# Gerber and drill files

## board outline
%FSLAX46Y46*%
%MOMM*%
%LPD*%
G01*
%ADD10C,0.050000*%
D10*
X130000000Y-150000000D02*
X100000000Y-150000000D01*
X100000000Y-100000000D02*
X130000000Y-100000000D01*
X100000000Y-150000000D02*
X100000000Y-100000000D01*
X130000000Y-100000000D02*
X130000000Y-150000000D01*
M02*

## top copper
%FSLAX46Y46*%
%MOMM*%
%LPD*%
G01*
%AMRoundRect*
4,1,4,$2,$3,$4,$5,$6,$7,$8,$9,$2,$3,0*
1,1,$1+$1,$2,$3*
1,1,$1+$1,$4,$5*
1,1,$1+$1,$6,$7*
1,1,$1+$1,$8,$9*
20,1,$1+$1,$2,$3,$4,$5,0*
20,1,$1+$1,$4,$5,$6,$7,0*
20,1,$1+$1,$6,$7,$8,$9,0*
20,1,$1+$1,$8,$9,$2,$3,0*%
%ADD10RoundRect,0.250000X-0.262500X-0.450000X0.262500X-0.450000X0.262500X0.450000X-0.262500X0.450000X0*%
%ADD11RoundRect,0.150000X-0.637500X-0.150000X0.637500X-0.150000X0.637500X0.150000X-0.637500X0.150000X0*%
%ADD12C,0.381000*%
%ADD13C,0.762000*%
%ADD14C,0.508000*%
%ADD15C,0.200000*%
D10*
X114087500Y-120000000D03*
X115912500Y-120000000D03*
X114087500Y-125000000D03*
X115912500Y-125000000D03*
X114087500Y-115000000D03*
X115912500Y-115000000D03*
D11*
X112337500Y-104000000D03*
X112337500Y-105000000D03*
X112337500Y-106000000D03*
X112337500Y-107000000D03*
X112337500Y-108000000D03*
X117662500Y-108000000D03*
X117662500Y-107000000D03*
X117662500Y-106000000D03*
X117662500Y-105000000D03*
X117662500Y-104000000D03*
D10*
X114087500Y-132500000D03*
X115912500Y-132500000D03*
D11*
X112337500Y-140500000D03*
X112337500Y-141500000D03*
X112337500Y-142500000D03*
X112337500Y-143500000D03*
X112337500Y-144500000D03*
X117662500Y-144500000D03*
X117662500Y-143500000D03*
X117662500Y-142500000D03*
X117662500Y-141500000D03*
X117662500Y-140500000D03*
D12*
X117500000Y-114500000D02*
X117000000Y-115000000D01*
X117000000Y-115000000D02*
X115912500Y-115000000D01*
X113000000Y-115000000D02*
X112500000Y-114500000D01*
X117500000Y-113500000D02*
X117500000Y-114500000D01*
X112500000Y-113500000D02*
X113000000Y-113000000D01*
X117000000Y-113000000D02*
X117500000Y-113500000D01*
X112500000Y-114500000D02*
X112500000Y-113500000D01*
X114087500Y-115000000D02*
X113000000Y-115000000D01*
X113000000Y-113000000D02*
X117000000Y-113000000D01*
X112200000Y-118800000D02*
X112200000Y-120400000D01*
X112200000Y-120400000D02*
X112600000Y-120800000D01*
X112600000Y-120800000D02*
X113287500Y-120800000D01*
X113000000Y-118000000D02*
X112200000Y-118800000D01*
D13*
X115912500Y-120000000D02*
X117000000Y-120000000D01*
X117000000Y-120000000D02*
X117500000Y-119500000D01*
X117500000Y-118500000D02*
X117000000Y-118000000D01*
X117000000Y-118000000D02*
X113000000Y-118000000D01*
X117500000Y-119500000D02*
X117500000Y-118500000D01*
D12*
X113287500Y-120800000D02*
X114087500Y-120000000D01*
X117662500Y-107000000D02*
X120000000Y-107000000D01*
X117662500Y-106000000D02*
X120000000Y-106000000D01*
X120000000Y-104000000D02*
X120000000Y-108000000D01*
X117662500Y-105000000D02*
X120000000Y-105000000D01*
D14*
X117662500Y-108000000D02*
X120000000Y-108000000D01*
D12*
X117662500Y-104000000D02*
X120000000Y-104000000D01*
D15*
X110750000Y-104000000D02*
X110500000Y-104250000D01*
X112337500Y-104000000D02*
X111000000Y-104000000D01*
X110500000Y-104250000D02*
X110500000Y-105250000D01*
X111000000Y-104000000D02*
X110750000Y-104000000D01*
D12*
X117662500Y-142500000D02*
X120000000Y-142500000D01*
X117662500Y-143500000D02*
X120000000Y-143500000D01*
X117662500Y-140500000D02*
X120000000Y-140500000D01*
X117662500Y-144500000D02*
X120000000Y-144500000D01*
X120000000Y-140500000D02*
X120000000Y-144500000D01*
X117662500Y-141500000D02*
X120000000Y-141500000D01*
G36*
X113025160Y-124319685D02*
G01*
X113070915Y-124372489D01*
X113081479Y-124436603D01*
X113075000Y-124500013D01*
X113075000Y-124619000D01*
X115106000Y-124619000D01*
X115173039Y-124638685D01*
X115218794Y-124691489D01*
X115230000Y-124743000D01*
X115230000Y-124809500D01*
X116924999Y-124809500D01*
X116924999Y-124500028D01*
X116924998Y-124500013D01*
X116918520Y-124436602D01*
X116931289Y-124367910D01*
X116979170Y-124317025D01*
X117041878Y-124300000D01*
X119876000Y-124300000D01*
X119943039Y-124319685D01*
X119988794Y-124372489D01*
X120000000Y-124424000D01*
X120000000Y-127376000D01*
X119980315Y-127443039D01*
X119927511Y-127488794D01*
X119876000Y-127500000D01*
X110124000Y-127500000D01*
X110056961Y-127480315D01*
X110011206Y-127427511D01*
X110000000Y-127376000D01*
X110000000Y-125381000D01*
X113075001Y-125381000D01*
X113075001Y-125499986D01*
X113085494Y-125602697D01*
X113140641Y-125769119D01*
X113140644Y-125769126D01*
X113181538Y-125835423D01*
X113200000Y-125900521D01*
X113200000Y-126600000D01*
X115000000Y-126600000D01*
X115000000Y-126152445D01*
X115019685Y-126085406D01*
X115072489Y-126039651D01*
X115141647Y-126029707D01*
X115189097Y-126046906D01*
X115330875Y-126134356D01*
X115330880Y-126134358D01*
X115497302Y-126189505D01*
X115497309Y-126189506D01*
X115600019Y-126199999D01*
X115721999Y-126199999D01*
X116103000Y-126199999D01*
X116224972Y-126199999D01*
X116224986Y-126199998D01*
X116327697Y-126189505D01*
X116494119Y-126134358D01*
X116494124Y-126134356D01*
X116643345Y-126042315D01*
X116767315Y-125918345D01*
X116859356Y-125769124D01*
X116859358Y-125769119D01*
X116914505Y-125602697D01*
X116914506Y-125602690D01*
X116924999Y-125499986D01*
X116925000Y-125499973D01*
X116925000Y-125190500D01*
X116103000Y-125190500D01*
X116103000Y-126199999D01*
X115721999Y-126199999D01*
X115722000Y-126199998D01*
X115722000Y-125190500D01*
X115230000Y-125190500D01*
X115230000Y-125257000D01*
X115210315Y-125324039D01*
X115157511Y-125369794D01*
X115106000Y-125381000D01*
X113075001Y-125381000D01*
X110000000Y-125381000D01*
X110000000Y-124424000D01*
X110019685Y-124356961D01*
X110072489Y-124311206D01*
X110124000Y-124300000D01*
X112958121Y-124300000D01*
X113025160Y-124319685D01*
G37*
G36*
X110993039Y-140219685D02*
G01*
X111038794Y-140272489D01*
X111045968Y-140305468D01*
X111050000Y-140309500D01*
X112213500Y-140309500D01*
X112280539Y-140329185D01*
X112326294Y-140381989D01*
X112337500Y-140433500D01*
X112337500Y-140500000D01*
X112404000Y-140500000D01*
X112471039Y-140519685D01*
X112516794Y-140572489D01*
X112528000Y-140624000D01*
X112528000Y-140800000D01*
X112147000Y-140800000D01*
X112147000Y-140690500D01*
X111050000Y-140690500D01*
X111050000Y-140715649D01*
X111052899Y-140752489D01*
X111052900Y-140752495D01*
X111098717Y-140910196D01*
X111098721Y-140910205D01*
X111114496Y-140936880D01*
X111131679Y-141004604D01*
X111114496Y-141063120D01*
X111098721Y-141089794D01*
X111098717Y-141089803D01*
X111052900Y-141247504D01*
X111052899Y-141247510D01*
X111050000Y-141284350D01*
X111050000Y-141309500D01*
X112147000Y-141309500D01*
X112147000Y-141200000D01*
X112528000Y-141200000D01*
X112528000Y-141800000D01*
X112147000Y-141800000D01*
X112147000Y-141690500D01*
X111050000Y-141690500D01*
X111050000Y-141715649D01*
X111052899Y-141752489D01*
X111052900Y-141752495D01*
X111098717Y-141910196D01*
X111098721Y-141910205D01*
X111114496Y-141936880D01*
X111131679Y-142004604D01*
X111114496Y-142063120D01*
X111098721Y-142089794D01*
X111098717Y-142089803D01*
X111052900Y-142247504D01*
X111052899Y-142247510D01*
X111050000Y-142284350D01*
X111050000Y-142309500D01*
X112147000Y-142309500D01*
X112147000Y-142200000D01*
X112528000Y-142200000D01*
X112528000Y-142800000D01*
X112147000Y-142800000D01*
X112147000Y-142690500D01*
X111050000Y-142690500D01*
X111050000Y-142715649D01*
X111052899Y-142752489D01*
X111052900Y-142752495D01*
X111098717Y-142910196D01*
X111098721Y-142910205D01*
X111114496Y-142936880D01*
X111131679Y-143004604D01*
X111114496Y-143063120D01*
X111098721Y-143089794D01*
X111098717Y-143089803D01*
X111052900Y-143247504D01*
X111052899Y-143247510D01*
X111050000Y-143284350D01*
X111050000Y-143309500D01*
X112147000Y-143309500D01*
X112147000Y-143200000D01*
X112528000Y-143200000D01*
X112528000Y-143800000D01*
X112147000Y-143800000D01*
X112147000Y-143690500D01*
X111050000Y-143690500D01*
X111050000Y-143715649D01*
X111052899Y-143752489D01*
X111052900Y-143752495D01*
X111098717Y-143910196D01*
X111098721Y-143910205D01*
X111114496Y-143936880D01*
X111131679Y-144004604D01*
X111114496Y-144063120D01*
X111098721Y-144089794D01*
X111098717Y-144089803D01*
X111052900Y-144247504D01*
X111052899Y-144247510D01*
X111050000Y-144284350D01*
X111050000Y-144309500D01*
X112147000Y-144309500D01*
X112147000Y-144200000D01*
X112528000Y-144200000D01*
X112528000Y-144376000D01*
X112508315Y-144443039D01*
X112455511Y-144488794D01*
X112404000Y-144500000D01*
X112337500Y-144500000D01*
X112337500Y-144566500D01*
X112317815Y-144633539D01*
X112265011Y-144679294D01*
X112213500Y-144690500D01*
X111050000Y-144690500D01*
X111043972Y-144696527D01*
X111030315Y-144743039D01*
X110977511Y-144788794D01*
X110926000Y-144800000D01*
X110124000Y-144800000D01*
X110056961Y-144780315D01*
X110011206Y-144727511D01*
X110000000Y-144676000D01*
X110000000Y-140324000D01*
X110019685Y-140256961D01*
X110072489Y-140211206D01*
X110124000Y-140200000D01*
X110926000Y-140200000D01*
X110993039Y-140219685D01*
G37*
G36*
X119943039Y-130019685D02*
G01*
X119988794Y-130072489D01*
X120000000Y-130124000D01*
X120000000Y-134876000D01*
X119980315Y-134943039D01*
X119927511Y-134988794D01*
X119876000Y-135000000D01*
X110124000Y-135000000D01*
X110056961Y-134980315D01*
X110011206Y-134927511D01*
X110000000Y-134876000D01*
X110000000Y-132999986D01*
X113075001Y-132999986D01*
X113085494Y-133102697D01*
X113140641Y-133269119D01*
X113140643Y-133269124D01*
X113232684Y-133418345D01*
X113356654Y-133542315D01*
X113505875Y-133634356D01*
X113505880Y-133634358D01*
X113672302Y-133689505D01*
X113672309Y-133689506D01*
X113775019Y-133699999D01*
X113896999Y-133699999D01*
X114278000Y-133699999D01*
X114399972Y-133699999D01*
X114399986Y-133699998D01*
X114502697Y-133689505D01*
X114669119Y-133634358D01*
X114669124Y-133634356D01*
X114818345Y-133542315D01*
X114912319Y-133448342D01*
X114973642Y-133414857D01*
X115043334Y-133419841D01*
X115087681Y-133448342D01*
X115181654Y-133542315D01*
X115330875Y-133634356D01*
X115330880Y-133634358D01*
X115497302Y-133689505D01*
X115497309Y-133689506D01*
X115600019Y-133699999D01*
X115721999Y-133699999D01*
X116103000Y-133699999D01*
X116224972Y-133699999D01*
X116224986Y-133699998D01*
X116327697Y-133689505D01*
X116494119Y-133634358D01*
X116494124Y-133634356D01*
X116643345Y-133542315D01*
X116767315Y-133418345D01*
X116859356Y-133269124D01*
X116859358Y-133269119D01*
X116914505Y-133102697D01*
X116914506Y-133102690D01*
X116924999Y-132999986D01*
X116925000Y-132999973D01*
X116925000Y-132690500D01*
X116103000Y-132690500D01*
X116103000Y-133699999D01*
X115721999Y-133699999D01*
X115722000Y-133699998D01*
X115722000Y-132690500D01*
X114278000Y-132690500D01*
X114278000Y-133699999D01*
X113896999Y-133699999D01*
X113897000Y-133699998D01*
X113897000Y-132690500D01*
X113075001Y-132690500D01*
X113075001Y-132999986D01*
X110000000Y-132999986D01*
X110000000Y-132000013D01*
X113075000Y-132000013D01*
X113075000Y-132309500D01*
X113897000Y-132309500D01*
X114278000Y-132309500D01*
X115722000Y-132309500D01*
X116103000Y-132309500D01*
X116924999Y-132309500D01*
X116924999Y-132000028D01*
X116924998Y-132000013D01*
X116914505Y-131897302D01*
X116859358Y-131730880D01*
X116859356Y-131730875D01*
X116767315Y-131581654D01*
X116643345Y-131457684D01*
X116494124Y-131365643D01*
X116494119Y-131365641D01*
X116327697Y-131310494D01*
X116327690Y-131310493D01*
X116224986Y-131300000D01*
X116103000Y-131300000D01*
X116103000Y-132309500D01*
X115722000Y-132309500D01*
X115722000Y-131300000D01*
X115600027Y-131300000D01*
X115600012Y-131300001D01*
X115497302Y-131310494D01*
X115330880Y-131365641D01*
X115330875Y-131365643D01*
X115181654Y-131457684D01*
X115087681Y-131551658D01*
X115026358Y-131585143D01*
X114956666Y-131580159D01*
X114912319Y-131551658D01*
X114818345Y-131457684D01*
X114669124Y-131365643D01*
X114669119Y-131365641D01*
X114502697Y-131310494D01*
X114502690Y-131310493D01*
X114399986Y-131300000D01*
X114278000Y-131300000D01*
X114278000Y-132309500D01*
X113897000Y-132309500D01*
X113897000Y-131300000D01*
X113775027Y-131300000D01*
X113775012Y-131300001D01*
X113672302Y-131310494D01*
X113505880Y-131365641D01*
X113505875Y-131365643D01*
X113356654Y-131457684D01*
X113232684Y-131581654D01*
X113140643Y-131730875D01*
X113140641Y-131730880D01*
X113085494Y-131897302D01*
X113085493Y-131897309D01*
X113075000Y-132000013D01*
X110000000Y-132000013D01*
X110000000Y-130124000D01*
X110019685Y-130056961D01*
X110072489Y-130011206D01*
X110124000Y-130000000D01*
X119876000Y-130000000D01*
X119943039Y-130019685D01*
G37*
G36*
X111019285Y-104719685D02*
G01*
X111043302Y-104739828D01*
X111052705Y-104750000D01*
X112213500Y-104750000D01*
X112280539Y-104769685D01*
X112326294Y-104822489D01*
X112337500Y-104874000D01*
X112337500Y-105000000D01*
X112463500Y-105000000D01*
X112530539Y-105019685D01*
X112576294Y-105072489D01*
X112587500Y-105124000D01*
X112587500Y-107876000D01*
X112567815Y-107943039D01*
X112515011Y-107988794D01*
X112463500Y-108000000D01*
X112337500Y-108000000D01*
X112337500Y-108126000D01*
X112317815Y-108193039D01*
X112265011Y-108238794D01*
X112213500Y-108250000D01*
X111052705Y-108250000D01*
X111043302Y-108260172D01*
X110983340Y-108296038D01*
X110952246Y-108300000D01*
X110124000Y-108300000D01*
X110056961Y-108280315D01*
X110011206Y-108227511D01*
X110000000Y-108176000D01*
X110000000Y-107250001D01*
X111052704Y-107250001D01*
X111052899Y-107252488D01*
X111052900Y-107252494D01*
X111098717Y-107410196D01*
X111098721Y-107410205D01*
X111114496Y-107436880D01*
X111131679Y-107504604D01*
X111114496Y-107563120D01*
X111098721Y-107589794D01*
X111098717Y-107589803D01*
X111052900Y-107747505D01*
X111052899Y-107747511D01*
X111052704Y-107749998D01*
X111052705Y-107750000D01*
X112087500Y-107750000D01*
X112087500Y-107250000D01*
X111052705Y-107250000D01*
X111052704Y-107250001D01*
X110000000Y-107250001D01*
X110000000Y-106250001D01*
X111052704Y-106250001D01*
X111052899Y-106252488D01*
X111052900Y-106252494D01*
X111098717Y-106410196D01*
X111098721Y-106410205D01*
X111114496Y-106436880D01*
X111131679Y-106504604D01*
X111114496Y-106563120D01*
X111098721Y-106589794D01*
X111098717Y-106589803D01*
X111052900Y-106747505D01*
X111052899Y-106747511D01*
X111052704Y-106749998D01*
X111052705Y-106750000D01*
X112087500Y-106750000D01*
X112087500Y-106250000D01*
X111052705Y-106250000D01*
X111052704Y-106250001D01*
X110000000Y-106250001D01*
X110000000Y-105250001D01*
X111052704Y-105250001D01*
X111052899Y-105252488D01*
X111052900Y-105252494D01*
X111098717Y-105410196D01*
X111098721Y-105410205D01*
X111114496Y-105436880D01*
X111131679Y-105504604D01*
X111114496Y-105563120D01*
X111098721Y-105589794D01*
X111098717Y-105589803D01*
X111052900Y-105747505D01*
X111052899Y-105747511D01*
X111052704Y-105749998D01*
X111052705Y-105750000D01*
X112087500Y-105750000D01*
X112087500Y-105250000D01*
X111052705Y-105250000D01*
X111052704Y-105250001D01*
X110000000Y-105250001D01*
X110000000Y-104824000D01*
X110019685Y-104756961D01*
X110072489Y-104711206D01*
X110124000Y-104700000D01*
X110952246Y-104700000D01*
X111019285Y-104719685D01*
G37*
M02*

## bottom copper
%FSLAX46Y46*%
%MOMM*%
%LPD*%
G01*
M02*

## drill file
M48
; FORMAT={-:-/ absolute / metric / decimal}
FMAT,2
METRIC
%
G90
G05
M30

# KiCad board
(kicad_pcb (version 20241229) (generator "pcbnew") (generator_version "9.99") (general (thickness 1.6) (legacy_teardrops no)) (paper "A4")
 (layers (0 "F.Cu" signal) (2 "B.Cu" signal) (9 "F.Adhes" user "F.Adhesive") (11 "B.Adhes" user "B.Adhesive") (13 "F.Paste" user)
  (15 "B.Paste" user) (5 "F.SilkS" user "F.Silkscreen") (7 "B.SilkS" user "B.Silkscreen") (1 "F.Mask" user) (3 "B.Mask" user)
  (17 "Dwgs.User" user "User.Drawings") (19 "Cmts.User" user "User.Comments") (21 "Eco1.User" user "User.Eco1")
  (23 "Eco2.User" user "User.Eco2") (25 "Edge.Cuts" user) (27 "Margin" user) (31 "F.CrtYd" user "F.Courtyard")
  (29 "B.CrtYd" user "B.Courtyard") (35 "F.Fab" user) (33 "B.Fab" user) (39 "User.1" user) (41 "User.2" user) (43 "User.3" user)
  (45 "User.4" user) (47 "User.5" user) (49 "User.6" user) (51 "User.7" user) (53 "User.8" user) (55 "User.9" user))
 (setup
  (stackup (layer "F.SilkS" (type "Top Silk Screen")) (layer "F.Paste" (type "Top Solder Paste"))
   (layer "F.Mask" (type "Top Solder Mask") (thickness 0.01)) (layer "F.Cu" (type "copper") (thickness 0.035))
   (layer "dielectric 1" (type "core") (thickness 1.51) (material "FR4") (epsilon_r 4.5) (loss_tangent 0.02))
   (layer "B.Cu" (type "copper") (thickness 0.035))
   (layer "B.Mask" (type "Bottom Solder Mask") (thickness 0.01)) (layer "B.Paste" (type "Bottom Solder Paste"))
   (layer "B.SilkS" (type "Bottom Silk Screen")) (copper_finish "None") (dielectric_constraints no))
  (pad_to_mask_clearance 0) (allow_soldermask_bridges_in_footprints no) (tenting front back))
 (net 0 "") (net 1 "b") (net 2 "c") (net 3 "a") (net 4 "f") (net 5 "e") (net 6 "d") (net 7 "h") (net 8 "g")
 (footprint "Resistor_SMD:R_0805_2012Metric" (layer "F.Cu") (at 115 120)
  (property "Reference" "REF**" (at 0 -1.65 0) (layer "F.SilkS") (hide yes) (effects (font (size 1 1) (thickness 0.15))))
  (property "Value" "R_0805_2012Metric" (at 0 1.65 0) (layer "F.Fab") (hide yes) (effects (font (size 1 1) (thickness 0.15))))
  (pad "1" smd roundrect (at -0.9125 0) (size 1.025 1.4) (layers "F.Cu" "F.Mask" "F.Paste") (roundrect_rratio 0.243902) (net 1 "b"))
  (pad "2" smd roundrect (at 0.9125 0) (size 1.025 1.4) (layers "F.Cu" "F.Mask" "F.Paste") (roundrect_rratio 0.243902) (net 1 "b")))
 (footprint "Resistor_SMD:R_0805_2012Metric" (layer "F.Cu") (at 115 125)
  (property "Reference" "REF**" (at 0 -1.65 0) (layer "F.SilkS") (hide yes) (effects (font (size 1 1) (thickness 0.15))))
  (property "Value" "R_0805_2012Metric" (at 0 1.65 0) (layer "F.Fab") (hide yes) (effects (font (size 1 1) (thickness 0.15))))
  (pad "1" smd roundrect (at -0.9125 0) (size 1.025 1.4) (layers "F.Cu" "F.Mask" "F.Paste") (roundrect_rratio 0.243902) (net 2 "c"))
  (pad "2" smd roundrect (at 0.9125 0) (size 1.025 1.4) (layers "F.Cu" "F.Mask" "F.Paste") (roundrect_rratio 0.243902) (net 2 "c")
   (thermal_bridge_width 0.381)))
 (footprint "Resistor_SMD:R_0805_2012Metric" (layer "F.Cu") (at 115 115)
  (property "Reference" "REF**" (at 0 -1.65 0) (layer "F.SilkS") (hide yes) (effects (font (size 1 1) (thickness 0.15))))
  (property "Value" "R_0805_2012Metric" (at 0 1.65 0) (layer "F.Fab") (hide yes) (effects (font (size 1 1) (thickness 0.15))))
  (pad "1" smd roundrect (at -0.9125 0) (size 1.025 1.4) (layers "F.Cu" "F.Mask" "F.Paste") (roundrect_rratio 0.243902) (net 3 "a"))
  (pad "2" smd roundrect (at 0.9125 0) (size 1.025 1.4) (layers "F.Cu" "F.Mask" "F.Paste") (roundrect_rratio 0.243902) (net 3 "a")))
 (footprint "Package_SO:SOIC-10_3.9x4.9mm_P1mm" (layer "F.Cu") (at 115 106)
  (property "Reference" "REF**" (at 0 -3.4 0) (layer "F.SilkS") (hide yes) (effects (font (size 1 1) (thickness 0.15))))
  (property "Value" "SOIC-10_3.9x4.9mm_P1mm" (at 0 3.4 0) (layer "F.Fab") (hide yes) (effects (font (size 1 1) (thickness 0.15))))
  (pad "1" smd roundrect (at -2.6625 -2) (size 1.575 0.6) (layers "F.Cu" "F.Mask" "F.Paste") (roundrect_rratio 0.25) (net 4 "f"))
  (pad "2" smd roundrect (at -2.6625 -1) (size 1.575 0.6) (layers "F.Cu" "F.Mask" "F.Paste") (roundrect_rratio 0.25) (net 4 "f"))
  (pad "3" smd roundrect (at -2.6625 0) (size 1.575 0.6) (layers "F.Cu" "F.Mask" "F.Paste") (roundrect_rratio 0.25) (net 4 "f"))
  (pad "4" smd roundrect (at -2.6625 1) (size 1.575 0.6) (layers "F.Cu" "F.Mask" "F.Paste") (roundrect_rratio 0.25) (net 4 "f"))
  (pad "5" smd roundrect (at -2.6625 2) (size 1.575 0.6) (layers "F.Cu" "F.Mask" "F.Paste") (roundrect_rratio 0.25) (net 4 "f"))
  (pad "6" smd roundrect (at 2.6625 2) (size 1.575 0.6) (layers "F.Cu" "F.Mask" "F.Paste") (roundrect_rratio 0.25) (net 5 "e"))
  (pad "7" smd roundrect (at 2.6625 1) (size 1.575 0.6) (layers "F.Cu" "F.Mask" "F.Paste") (roundrect_rratio 0.25) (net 5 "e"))
  (pad "8" smd roundrect (at 2.6625 0) (size 1.575 0.6) (layers "F.Cu" "F.Mask" "F.Paste") (roundrect_rratio 0.25) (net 5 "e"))
  (pad "9" smd roundrect (at 2.6625 -1) (size 1.575 0.6) (layers "F.Cu" "F.Mask" "F.Paste") (roundrect_rratio 0.25) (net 5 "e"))
  (pad "10" smd roundrect (at 2.6625 -2) (size 1.575 0.6) (layers "F.Cu" "F.Mask" "F.Paste") (roundrect_rratio 0.25) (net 5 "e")))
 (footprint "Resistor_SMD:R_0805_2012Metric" (layer "F.Cu") (at 115 132.5)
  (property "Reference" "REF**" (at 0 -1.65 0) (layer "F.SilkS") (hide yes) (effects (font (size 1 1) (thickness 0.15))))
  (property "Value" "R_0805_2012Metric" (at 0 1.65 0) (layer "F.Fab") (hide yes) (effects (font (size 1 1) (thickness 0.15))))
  (pad "1" smd roundrect (at -0.9125 0) (size 1.025 1.4) (layers "F.Cu" "F.Mask" "F.Paste") (roundrect_rratio 0.243902) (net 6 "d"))
  (pad "2" smd roundrect (at 0.9125 0) (size 1.025 1.4) (layers "F.Cu" "F.Mask" "F.Paste") (roundrect_rratio 0.243902) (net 6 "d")))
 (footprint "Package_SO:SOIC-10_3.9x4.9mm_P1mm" (layer "F.Cu") (at 115 142.5)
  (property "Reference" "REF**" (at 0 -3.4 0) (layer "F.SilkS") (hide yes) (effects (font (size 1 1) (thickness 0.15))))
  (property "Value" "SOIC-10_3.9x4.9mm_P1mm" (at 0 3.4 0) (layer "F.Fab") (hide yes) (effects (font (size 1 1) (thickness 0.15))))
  (pad "1" smd roundrect (at -2.6625 -2) (size 1.575 0.6) (layers "F.Cu" "F.Mask" "F.Paste") (roundrect_rratio 0.25) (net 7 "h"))
  (pad "2" smd roundrect (at -2.6625 -1) (size 1.575 0.6) (layers "F.Cu" "F.Mask" "F.Paste") (roundrect_rratio 0.25) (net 7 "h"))
  (pad "3" smd roundrect (at -2.6625 0) (size 1.575 0.6) (layers "F.Cu" "F.Mask" "F.Paste") (roundrect_rratio 0.25) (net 7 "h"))
  (pad "4" smd roundrect (at -2.6625 1) (size 1.575 0.6) (layers "F.Cu" "F.Mask" "F.Paste") (roundrect_rratio 0.25) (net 7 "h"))
  (pad "5" smd roundrect (at -2.6625 2) (size 1.575 0.6) (layers "F.Cu" "F.Mask" "F.Paste") (roundrect_rratio 0.25) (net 7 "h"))
  (pad "6" smd roundrect (at 2.6625 2) (size 1.575 0.6) (layers "F.Cu" "F.Mask" "F.Paste") (roundrect_rratio 0.25) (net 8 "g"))
  (pad "7" smd roundrect (at 2.6625 1) (size 1.575 0.6) (layers "F.Cu" "F.Mask" "F.Paste") (roundrect_rratio 0.25) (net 8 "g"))
  (pad "8" smd roundrect (at 2.6625 0) (size 1.575 0.6) (layers "F.Cu" "F.Mask" "F.Paste") (roundrect_rratio 0.25) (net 8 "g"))
  (pad "9" smd roundrect (at 2.6625 -1) (size 1.575 0.6) (layers "F.Cu" "F.Mask" "F.Paste") (roundrect_rratio 0.25) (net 8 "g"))
  (pad "10" smd roundrect (at 2.6625 -2) (size 1.575 0.6) (layers "F.Cu" "F.Mask" "F.Paste") (roundrect_rratio 0.25) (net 8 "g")))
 (gr_line (start 130 150) (end 100 150) (stroke (width 0.05) (type default)) (layer "Edge.Cuts"))
 (gr_line (start 100 100) (end 130 100) (stroke (width 0.05) (type default)) (layer "Edge.Cuts"))
 (gr_line (start 100 150) (end 100 100) (stroke (width 0.05) (type default)) (layer "Edge.Cuts"))
 (gr_line (start 130 100) (end 130 150) (stroke (width 0.05) (type default)) (layer "Edge.Cuts"))
 (segment (start 117.5 114.5) (end 117 115) (width 0.381) (layer "F.Cu") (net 3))
 (segment (start 117 115) (end 115.9125 115) (width 0.381) (layer "F.Cu") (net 3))
 (segment (start 113 115) (end 112.5 114.5) (width 0.381) (layer "F.Cu") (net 3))
 (segment (start 117.5 113.5) (end 117.5 114.5) (width 0.381) (layer "F.Cu") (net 3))
 (segment (start 112.5 113.5) (end 113 113) (width 0.381) (layer "F.Cu") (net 3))
 (segment (start 117 113) (end 117.5 113.5) (width 0.381) (layer "F.Cu") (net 3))
 (segment (start 112.5 114.5) (end 112.5 113.5) (width 0.381) (layer "F.Cu") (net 3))
 (segment (start 114.0875 115) (end 113 115) (width 0.381) (layer "F.Cu") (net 3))
 (segment (start 113 113) (end 117 113) (width 0.381) (layer "F.Cu") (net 3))
 (segment (start 112.2 118.8) (end 112.2 120.4) (width 0.381) (layer "F.Cu") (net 1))
 (segment (start 112.2 120.4) (end 112.6 120.8) (width 0.381) (layer "F.Cu") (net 1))
 (segment (start 112.6 120.8) (end 113.2875 120.8) (width 0.381) (layer "F.Cu") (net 1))
 (segment (start 113 118) (end 112.2 118.8) (width 0.381) (layer "F.Cu") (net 1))
 (segment (start 115.9125 120) (end 117 120) (width 0.762) (layer "F.Cu") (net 1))
 (segment (start 117 120) (end 117.5 119.5) (width 0.762) (layer "F.Cu") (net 1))
 (segment (start 117.5 118.5) (end 117 118) (width 0.762) (layer "F.Cu") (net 1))
 (segment (start 117 118) (end 113 118) (width 0.762) (layer "F.Cu") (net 1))
 (segment (start 117.5 119.5) (end 117.5 118.5) (width 0.762) (layer "F.Cu") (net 1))
 (segment (start 113.2875 120.8) (end 114.0875 120) (width 0.381) (layer "F.Cu") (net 1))
 (segment (start 117.6625 107) (end 120 107) (width 0.381) (layer "F.Cu") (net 5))
 (segment (start 117.6625 106) (end 120 106) (width 0.381) (layer "F.Cu") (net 5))
 (segment (start 120 104) (end 120 108) (width 0.381) (layer "F.Cu") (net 5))
 (segment (start 117.6625 105) (end 120 105) (width 0.381) (layer "F.Cu") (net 5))
 (segment (start 117.6625 108) (end 120 108) (width 0.508) (layer "F.Cu") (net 5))
 (segment (start 117.6625 104) (end 120 104) (width 0.381) (layer "F.Cu") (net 5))
 (segment (start 110.75 104) (end 110.5 104.25) (width 0.2) (layer "F.Cu") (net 4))
 (segment (start 112.3375 104) (end 111 104) (width 0.2) (layer "F.Cu") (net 4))
 (segment (start 110.5 104.25) (end 110.5 105.25) (width 0.2) (layer "F.Cu") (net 4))
 (segment (start 111 104) (end 110.75 104) (width 0.2) (layer "F.Cu") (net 4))
 (segment (start 117.6625 142.5) (end 120 142.5) (width 0.381) (layer "F.Cu") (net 8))
 (segment (start 117.6625 143.5) (end 120 143.5) (width 0.381) (layer "F.Cu") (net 8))
 (segment (start 117.6625 140.5) (end 120 140.5) (width 0.381) (layer "F.Cu") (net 8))
 (segment (start 117.6625 144.5) (end 120 144.5) (width 0.381) (layer "F.Cu") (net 8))
 (segment (start 120 140.5) (end 120 144.5) (width 0.381) (layer "F.Cu") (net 8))
 (segment (start 117.6625 141.5) (end 120 141.5) (width 0.381) (layer "F.Cu") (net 8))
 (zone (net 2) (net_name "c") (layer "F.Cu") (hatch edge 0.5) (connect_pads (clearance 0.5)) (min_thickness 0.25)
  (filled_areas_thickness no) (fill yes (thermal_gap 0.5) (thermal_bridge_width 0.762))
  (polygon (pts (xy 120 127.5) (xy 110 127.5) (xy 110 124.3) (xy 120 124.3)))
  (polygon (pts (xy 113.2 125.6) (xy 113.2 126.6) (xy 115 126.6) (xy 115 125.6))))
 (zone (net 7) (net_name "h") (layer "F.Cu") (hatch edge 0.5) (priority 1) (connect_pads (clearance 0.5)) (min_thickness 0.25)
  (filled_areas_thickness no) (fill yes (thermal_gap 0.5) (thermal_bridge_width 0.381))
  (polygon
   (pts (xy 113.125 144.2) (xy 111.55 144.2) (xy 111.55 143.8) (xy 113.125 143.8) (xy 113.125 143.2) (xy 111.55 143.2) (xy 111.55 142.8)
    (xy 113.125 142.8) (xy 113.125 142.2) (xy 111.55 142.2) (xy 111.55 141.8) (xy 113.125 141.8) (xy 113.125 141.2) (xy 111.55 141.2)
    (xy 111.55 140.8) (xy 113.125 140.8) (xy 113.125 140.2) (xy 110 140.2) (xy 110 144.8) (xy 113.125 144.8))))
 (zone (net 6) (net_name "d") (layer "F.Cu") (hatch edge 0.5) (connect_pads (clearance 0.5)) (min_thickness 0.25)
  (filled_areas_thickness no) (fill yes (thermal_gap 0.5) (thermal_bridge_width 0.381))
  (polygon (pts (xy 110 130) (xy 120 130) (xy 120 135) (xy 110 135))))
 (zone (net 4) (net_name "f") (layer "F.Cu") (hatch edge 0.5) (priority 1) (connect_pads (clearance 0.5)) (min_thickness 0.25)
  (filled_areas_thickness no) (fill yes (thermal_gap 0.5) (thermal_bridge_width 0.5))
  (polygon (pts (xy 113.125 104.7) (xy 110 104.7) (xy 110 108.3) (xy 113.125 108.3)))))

